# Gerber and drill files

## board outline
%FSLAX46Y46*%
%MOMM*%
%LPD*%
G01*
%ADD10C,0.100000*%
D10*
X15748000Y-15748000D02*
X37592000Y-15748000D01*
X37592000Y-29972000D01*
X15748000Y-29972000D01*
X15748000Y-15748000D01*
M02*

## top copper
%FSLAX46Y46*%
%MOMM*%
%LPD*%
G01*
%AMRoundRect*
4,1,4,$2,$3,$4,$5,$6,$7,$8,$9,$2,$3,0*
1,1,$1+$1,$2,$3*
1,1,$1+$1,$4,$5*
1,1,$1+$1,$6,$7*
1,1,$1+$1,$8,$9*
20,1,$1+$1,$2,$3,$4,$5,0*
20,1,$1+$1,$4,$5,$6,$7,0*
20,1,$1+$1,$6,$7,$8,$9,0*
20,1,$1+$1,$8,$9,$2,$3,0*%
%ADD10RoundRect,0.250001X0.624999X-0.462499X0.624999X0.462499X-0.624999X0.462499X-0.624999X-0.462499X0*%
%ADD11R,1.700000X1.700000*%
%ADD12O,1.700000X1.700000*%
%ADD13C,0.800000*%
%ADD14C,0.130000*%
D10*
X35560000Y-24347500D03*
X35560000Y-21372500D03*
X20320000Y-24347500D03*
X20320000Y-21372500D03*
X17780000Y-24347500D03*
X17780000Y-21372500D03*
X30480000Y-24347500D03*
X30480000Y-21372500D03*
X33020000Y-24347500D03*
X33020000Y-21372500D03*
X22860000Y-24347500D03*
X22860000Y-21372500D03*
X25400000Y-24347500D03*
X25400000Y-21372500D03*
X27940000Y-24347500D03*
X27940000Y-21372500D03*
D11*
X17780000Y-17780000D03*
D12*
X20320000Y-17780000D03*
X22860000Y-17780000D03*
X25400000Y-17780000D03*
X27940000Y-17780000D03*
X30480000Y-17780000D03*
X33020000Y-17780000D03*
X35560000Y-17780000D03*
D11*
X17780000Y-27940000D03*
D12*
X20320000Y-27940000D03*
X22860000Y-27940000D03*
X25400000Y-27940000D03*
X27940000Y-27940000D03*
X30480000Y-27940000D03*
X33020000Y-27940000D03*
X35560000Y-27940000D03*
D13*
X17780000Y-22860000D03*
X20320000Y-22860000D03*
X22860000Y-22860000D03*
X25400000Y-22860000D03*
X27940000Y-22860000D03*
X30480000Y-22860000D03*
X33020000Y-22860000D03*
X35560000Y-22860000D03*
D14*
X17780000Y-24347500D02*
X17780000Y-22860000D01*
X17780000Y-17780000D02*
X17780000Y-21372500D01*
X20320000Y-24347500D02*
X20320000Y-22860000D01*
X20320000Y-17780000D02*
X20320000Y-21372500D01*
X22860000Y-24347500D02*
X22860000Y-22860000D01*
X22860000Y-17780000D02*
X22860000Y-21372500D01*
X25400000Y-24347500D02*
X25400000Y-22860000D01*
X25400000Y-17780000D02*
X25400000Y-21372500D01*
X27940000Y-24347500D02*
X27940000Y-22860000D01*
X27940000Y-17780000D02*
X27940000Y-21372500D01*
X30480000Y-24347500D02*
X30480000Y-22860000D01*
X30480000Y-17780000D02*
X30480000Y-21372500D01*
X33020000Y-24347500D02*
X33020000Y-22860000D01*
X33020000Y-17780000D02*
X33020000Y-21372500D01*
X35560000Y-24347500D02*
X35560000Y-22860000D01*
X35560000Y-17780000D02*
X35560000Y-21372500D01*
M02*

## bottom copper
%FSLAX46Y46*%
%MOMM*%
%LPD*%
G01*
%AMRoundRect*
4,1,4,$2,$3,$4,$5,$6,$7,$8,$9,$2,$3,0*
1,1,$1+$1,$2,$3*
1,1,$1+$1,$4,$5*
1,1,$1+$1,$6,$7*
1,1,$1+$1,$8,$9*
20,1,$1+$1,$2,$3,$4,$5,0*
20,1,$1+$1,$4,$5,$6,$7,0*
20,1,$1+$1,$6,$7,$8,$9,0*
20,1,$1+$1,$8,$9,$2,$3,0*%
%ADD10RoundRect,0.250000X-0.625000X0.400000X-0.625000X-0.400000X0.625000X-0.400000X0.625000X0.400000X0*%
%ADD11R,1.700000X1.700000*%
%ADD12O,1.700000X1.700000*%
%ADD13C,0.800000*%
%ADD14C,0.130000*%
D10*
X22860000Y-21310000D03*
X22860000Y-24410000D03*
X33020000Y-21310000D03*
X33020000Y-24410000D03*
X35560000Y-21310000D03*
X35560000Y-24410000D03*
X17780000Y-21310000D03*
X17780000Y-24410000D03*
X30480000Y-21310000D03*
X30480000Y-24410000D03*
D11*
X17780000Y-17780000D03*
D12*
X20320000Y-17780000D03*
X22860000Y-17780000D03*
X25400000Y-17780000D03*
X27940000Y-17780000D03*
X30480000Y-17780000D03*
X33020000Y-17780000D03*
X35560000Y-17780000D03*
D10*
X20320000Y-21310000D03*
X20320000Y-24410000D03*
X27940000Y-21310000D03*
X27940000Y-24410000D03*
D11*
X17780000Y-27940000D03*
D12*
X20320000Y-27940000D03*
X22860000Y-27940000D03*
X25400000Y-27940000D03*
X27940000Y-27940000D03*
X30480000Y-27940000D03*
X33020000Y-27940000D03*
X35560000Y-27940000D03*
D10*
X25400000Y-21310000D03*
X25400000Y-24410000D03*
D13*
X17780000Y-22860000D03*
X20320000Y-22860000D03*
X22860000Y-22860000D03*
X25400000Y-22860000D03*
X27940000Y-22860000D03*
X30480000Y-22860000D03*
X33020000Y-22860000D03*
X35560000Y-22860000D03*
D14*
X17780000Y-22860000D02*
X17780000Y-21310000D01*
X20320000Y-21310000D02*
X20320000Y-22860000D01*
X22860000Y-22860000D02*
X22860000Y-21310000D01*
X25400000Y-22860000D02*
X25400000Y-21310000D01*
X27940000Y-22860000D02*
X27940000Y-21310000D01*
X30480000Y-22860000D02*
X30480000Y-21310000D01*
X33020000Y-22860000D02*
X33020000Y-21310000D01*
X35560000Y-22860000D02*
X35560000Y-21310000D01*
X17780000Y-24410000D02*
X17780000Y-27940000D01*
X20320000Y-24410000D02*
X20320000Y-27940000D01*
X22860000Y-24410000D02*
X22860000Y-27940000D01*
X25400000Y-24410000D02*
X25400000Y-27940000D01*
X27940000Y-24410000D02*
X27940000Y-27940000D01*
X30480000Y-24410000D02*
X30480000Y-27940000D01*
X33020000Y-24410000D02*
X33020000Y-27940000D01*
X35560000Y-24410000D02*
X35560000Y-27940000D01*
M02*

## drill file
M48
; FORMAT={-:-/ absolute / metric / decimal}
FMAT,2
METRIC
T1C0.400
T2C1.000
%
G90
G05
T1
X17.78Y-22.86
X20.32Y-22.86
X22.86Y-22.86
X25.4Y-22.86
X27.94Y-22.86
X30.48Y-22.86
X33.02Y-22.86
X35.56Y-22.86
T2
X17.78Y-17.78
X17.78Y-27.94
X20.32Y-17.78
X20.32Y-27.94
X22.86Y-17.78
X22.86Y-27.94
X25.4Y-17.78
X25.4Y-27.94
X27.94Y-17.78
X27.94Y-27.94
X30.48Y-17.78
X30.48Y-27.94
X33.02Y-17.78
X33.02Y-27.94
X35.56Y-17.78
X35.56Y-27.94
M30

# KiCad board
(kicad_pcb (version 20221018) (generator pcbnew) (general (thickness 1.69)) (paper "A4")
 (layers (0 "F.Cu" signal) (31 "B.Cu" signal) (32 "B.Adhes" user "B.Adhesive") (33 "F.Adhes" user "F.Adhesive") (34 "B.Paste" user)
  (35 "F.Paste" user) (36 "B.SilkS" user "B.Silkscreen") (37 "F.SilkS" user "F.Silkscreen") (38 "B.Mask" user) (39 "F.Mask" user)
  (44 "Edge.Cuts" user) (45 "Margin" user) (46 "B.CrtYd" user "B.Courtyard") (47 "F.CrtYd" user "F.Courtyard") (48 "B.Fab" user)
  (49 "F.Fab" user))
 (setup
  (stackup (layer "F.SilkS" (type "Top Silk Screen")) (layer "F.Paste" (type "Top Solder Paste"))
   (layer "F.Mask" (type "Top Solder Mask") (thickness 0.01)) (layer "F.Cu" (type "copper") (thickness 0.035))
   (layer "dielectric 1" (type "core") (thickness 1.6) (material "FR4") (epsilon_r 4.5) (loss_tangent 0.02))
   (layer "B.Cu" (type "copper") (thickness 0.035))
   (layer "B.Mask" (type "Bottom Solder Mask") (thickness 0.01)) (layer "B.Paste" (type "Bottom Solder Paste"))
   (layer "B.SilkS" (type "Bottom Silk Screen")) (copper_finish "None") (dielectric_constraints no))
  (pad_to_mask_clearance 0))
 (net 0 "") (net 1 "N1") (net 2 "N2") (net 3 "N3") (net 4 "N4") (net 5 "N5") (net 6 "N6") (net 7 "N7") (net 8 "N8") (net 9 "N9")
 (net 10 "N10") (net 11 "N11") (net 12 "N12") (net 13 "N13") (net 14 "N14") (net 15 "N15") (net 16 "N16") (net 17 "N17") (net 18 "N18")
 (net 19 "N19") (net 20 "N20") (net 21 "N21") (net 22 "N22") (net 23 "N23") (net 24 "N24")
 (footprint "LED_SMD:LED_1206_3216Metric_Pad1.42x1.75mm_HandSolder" (layer "F.Cu") (at 35.56 22.86 90)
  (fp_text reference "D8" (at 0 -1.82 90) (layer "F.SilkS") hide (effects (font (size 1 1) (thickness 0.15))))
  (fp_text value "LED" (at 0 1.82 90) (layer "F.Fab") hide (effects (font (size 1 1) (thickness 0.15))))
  (pad "1" smd roundrect (at -1.4875 0 90) (size 1.425 1.75) (layers "F.Cu" "F.Paste" "F.Mask") (roundrect_rratio 0.1754392982) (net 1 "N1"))
  (pad "2" smd roundrect (at 1.4875 0 90) (size 1.425 1.75) (layers "F.Cu" "F.Paste" "F.Mask") (roundrect_rratio 0.1754392982) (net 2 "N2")))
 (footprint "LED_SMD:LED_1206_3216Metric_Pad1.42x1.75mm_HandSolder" (layer "F.Cu") (at 20.32 22.86 90)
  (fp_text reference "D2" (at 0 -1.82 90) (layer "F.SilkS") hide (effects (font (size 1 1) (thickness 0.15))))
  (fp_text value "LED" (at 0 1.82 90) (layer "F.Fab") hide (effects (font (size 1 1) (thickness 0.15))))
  (pad "1" smd roundrect (at -1.4875 0 90) (size 1.425 1.75) (layers "F.Cu" "F.Paste" "F.Mask") (roundrect_rratio 0.1754392982) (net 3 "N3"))
  (pad "2" smd roundrect (at 1.4875 0 90) (size 1.425 1.75) (layers "F.Cu" "F.Paste" "F.Mask") (roundrect_rratio 0.1754392982) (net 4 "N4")))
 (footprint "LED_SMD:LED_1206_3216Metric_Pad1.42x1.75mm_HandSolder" (layer "F.Cu") (at 17.78 22.86 90)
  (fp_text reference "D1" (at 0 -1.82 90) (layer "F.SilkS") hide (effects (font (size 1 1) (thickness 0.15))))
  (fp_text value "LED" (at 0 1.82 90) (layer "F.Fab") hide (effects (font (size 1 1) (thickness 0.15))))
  (pad "1" smd roundrect (at -1.4875 0 90) (size 1.425 1.75) (layers "F.Cu" "F.Paste" "F.Mask") (roundrect_rratio 0.1754392982) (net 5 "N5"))
  (pad "2" smd roundrect (at 1.4875 0 90) (size 1.425 1.75) (layers "F.Cu" "F.Paste" "F.Mask") (roundrect_rratio 0.1754392982) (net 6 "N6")))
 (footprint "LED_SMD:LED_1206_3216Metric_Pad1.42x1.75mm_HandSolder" (layer "F.Cu") (at 30.48 22.86 90)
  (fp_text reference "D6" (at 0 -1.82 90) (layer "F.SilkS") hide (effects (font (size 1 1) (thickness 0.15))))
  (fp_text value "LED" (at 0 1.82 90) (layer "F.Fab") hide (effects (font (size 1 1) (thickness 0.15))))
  (pad "1" smd roundrect (at -1.4875 0 90) (size 1.425 1.75) (layers "F.Cu" "F.Paste" "F.Mask") (roundrect_rratio 0.1754392982) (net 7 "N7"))
  (pad "2" smd roundrect (at 1.4875 0 90) (size 1.425 1.75) (layers "F.Cu" "F.Paste" "F.Mask") (roundrect_rratio 0.1754392982) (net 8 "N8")))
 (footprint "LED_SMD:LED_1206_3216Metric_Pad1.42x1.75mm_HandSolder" (layer "F.Cu") (at 33.02 22.86 90)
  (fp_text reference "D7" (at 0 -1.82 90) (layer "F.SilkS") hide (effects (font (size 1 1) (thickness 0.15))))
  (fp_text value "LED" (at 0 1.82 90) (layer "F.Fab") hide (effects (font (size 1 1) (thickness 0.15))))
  (pad "1" smd roundrect (at -1.4875 0 90) (size 1.425 1.75) (layers "F.Cu" "F.Paste" "F.Mask") (roundrect_rratio 0.1754392982) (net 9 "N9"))
  (pad "2" smd roundrect (at 1.4875 0 90) (size 1.425 1.75) (layers "F.Cu" "F.Paste" "F.Mask") (roundrect_rratio 0.1754392982)
   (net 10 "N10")))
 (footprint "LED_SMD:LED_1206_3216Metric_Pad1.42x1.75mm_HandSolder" (layer "F.Cu") (at 22.86 22.86 90)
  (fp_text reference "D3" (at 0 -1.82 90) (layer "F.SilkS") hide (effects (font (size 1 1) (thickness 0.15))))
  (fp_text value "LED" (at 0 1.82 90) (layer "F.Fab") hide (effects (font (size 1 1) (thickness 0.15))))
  (pad "1" smd roundrect (at -1.4875 0 90) (size 1.425 1.75) (layers "F.Cu" "F.Paste" "F.Mask") (roundrect_rratio 0.1754392982)
   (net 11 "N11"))
  (pad "2" smd roundrect (at 1.4875 0 90) (size 1.425 1.75) (layers "F.Cu" "F.Paste" "F.Mask") (roundrect_rratio 0.1754392982)
   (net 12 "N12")))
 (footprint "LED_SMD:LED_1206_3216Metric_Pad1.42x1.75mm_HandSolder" (layer "F.Cu") (at 25.4 22.86 90)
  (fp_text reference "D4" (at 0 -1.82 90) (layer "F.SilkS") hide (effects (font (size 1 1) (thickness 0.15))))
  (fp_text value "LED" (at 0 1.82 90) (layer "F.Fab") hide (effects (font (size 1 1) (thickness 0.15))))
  (pad "1" smd roundrect (at -1.4875 0 90) (size 1.425 1.75) (layers "F.Cu" "F.Paste" "F.Mask") (roundrect_rratio 0.1754392982)
   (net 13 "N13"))
  (pad "2" smd roundrect (at 1.4875 0 90) (size 1.425 1.75) (layers "F.Cu" "F.Paste" "F.Mask") (roundrect_rratio 0.1754392982)
   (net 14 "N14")))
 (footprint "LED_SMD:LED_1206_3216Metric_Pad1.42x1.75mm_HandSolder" (layer "F.Cu") (at 27.94 22.86 90)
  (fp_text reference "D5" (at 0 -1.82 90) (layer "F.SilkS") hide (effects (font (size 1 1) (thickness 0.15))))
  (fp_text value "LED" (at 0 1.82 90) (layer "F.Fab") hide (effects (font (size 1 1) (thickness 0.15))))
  (pad "1" smd roundrect (at -1.4875 0 90) (size 1.425 1.75) (layers "F.Cu" "F.Paste" "F.Mask") (roundrect_rratio 0.1754392982)
   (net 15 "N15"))
  (pad "2" smd roundrect (at 1.4875 0 90) (size 1.425 1.75) (layers "F.Cu" "F.Paste" "F.Mask") (roundrect_rratio 0.1754392982)
   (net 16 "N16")))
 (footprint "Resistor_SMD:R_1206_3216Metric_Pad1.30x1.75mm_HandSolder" (layer "B.Cu") (at 22.86 22.86 -90)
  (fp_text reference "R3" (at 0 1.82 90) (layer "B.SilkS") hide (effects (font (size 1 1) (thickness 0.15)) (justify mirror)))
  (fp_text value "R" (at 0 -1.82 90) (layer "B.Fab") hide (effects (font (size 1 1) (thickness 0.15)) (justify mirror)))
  (pad "1" smd roundrect (at -1.55 0 270) (size 1.3 1.75) (layers "B.Cu" "B.Paste" "B.Mask") (roundrect_rratio 0.1923076923) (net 11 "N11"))
  (pad "2" smd roundrect (at 1.55 0 270) (size 1.3 1.75) (layers "B.Cu" "B.Paste" "B.Mask") (roundrect_rratio 0.1923076923) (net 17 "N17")))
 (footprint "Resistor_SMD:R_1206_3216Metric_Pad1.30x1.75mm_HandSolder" (layer "B.Cu") (at 33.02 22.86 -90)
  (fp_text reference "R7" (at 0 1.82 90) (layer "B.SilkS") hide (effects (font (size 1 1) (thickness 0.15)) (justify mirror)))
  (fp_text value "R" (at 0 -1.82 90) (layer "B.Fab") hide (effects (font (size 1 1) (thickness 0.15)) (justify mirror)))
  (pad "1" smd roundrect (at -1.55 0 270) (size 1.3 1.75) (layers "B.Cu" "B.Paste" "B.Mask") (roundrect_rratio 0.1923076923) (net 9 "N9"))
  (pad "2" smd roundrect (at 1.55 0 270) (size 1.3 1.75) (layers "B.Cu" "B.Paste" "B.Mask") (roundrect_rratio 0.1923076923) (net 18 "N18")))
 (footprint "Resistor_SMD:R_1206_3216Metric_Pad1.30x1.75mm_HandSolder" (layer "B.Cu") (at 35.56 22.86 -90)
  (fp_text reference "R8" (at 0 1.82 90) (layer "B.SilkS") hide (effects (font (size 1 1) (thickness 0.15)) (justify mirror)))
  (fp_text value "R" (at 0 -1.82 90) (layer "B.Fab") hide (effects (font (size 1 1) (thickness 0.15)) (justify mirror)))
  (pad "1" smd roundrect (at -1.55 0 270) (size 1.3 1.75) (layers "B.Cu" "B.Paste" "B.Mask") (roundrect_rratio 0.1923076923) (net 1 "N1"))
  (pad "2" smd roundrect (at 1.55 0 270) (size 1.3 1.75) (layers "B.Cu" "B.Paste" "B.Mask") (roundrect_rratio 0.1923076923) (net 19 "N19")))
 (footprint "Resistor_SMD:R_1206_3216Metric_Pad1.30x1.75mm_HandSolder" (layer "B.Cu") (at 17.78 22.86 -90)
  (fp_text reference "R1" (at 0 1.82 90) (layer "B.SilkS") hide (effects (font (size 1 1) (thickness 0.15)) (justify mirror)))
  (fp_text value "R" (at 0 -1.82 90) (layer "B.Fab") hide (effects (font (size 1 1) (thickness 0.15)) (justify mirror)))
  (pad "1" smd roundrect (at -1.55 0 270) (size 1.3 1.75) (layers "B.Cu" "B.Paste" "B.Mask") (roundrect_rratio 0.1923076923) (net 5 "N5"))
  (pad "2" smd roundrect (at 1.55 0 270) (size 1.3 1.75) (layers "B.Cu" "B.Paste" "B.Mask") (roundrect_rratio 0.1923076923) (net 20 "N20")))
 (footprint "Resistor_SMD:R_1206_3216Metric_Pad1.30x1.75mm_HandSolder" (layer "B.Cu") (at 30.48 22.86 -90)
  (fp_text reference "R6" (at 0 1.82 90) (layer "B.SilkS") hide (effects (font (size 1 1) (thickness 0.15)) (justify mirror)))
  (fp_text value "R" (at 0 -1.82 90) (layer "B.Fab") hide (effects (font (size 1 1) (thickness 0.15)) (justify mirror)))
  (pad "1" smd roundrect (at -1.55 0 270) (size 1.3 1.75) (layers "B.Cu" "B.Paste" "B.Mask") (roundrect_rratio 0.1923076923) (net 7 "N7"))
  (pad "2" smd roundrect (at 1.55 0 270) (size 1.3 1.75) (layers "B.Cu" "B.Paste" "B.Mask") (roundrect_rratio 0.1923076923) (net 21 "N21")))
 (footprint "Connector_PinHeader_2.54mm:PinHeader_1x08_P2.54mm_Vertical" (layer "B.Cu") (at 17.78 17.78 -90)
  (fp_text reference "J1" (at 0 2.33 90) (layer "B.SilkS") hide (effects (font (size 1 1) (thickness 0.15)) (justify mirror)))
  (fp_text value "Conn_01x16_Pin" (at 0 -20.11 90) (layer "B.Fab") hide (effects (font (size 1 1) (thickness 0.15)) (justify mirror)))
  (pad "1" thru_hole rect (at 0 0 270) (size 1.7 1.7) (drill 1) (layers "*.Cu" "*.Mask") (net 6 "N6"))
  (pad "2" thru_hole oval (at 0 -2.54 270) (size 1.7 1.7) (drill 1) (layers "*.Cu" "*.Mask") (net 4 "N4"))
  (pad "3" thru_hole oval (at 0 -5.08 270) (size 1.7 1.7) (drill 1) (layers "*.Cu" "*.Mask") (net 12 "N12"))
  (pad "4" thru_hole oval (at 0 -7.62 270) (size 1.7 1.7) (drill 1) (layers "*.Cu" "*.Mask") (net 14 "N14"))
  (pad "5" thru_hole oval (at 0 -10.16 270) (size 1.7 1.7) (drill 1) (layers "*.Cu" "*.Mask") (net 16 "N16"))
  (pad "6" thru_hole oval (at 0 -12.7 270) (size 1.7 1.7) (drill 1) (layers "*.Cu" "*.Mask") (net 8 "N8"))
  (pad "7" thru_hole oval (at 0 -15.24 270) (size 1.7 1.7) (drill 1) (layers "*.Cu" "*.Mask") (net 10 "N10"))
  (pad "8" thru_hole oval (at 0 -17.78 270) (size 1.7 1.7) (drill 1) (layers "*.Cu" "*.Mask") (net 2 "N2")))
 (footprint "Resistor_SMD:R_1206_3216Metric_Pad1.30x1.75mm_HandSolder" (layer "B.Cu") (at 20.32 22.86 -90)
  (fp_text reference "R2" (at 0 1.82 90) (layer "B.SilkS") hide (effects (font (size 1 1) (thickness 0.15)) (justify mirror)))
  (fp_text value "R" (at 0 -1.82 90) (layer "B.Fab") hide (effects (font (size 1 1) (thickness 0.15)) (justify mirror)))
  (pad "1" smd roundrect (at -1.55 0 270) (size 1.3 1.75) (layers "B.Cu" "B.Paste" "B.Mask") (roundrect_rratio 0.1923076923) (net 3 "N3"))
  (pad "2" smd roundrect (at 1.55 0 270) (size 1.3 1.75) (layers "B.Cu" "B.Paste" "B.Mask") (roundrect_rratio 0.1923076923) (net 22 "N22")))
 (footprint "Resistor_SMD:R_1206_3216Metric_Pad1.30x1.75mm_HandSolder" (layer "B.Cu") (at 27.94 22.86 -90)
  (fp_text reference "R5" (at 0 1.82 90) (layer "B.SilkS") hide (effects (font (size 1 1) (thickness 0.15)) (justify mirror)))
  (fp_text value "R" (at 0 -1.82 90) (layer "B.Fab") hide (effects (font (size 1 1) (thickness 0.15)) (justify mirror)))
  (pad "1" smd roundrect (at -1.55 0 270) (size 1.3 1.75) (layers "B.Cu" "B.Paste" "B.Mask") (roundrect_rratio 0.1923076923) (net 15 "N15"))
  (pad "2" smd roundrect (at 1.55 0 270) (size 1.3 1.75) (layers "B.Cu" "B.Paste" "B.Mask") (roundrect_rratio 0.1923076923) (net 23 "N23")))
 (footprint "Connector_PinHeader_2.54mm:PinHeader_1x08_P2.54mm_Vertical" (layer "B.Cu") (at 17.78 27.94 -90)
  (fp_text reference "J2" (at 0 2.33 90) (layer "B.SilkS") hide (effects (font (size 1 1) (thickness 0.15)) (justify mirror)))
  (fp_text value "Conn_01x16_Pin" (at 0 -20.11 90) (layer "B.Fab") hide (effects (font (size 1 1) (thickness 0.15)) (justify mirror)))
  (pad "1" thru_hole rect (at 0 0 270) (size 1.7 1.7) (drill 1) (layers "*.Cu" "*.Mask") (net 20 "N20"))
  (pad "2" thru_hole oval (at 0 -2.54 270) (size 1.7 1.7) (drill 1) (layers "*.Cu" "*.Mask") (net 22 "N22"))
  (pad "3" thru_hole oval (at 0 -5.08 270) (size 1.7 1.7) (drill 1) (layers "*.Cu" "*.Mask") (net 17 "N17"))
  (pad "4" thru_hole oval (at 0 -7.62 270) (size 1.7 1.7) (drill 1) (layers "*.Cu" "*.Mask") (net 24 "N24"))
  (pad "5" thru_hole oval (at 0 -10.16 270) (size 1.7 1.7) (drill 1) (layers "*.Cu" "*.Mask") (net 23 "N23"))
  (pad "6" thru_hole oval (at 0 -12.7 270) (size 1.7 1.7) (drill 1) (layers "*.Cu" "*.Mask") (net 21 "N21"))
  (pad "7" thru_hole oval (at 0 -15.24 270) (size 1.7 1.7) (drill 1) (layers "*.Cu" "*.Mask") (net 18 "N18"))
  (pad "8" thru_hole oval (at 0 -17.78 270) (size 1.7 1.7) (drill 1) (layers "*.Cu" "*.Mask") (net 19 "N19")))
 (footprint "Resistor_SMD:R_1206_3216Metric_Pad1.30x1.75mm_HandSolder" (layer "B.Cu") (at 25.4 22.86 -90)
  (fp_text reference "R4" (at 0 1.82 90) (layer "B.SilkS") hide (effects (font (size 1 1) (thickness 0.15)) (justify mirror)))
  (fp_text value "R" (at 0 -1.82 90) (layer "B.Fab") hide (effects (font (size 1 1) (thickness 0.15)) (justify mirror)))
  (pad "1" smd roundrect (at -1.55 0 270) (size 1.3 1.75) (layers "B.Cu" "B.Paste" "B.Mask") (roundrect_rratio 0.1923076923) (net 13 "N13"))
  (pad "2" smd roundrect (at 1.55 0 270) (size 1.3 1.75) (layers "B.Cu" "B.Paste" "B.Mask") (roundrect_rratio 0.1923076923) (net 24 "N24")))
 (gr_rect (start 15.748 15.748) (end 37.592 29.972) (stroke (width 0.1) (type default)) (fill none) (layer "Edge.Cuts"))
 (segment (start 17.78 24.3475) (end 17.78 22.86) (width 0.13) (layer "F.Cu") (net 5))
 (via (at 17.78 22.86) (size 0.8) (drill 0.4) (layers "F.Cu" "B.Cu") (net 5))
 (segment (start 17.78 22.86) (end 17.78 21.31) (width 0.13) (layer "B.Cu") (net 5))
 (segment (start 17.78 17.78) (end 17.78 21.3725) (width 0.13) (layer "F.Cu") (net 6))
 (segment (start 20.32 24.3475) (end 20.32 22.86) (width 0.13) (layer "F.Cu") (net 3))
 (via (at 20.32 22.86) (size 0.8) (drill 0.4) (layers "F.Cu" "B.Cu") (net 3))
 (segment (start 20.32 21.31) (end 20.32 22.86) (width 0.13) (layer "B.Cu") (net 3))
 (segment (start 20.32 17.78) (end 20.32 21.3725) (width 0.13) (layer "F.Cu") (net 4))
 (segment (start 22.86 24.3475) (end 22.86 22.86) (width 0.13) (layer "F.Cu") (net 11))
 (via (at 22.86 22.86) (size 0.8) (drill 0.4) (layers "F.Cu" "B.Cu") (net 11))
 (segment (start 22.86 22.86) (end 22.86 21.31) (width 0.13) (layer "B.Cu") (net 11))
 (segment (start 22.86 17.78) (end 22.86 21.3725) (width 0.13) (layer "F.Cu") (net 12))
 (segment (start 25.4 24.3475) (end 25.4 22.86) (width 0.13) (layer "F.Cu") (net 13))
 (via (at 25.4 22.86) (size 0.8) (drill 0.4) (layers "F.Cu" "B.Cu") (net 13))
 (segment (start 25.4 22.86) (end 25.4 21.31) (width 0.13) (layer "B.Cu") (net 13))
 (segment (start 25.4 17.78) (end 25.4 21.3725) (width 0.13) (layer "F.Cu") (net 14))
 (segment (start 27.94 24.3475) (end 27.94 22.86) (width 0.13) (layer "F.Cu") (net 15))
 (via (at 27.94 22.86) (size 0.8) (drill 0.4) (layers "F.Cu" "B.Cu") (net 15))
 (segment (start 27.94 22.86) (end 27.94 21.31) (width 0.13) (layer "B.Cu") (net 15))
 (segment (start 27.94 17.78) (end 27.94 21.3725) (width 0.13) (layer "F.Cu") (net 16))
 (segment (start 30.48 24.3475) (end 30.48 22.86) (width 0.13) (layer "F.Cu") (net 7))
 (via (at 30.48 22.86) (size 0.8) (drill 0.4) (layers "F.Cu" "B.Cu") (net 7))
 (segment (start 30.48 22.86) (end 30.48 21.31) (width 0.13) (layer "B.Cu") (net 7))
 (segment (start 30.48 17.78) (end 30.48 21.3725) (width 0.13) (layer "F.Cu") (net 8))
 (segment (start 33.02 24.3475) (end 33.02 22.86) (width 0.13) (layer "F.Cu") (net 9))
 (via (at 33.02 22.86) (size 0.8) (drill 0.4) (layers "F.Cu" "B.Cu") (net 9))
 (segment (start 33.02 22.86) (end 33.02 21.31) (width 0.13) (layer "B.Cu") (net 9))
 (segment (start 33.02 17.78) (end 33.02 21.3725) (width 0.13) (layer "F.Cu") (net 10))
 (segment (start 35.56 24.3475) (end 35.56 22.86) (width 0.13) (layer "F.Cu") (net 1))
 (via (at 35.56 22.86) (size 0.8) (drill 0.4) (layers "F.Cu" "B.Cu") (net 1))
 (segment (start 35.56 22.86) (end 35.56 21.31) (width 0.13) (layer "B.Cu") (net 1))
 (segment (start 35.56 17.78) (end 35.56 21.3725) (width 0.13) (layer "F.Cu") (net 2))
 (segment (start 17.78 24.41) (end 17.78 27.94) (width 0.13) (layer "B.Cu") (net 20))
 (segment (start 20.32 24.41) (end 20.32 27.94) (width 0.13) (layer "B.Cu") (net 22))
 (segment (start 22.86 24.41) (end 22.86 27.94) (width 0.13) (layer "B.Cu") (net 17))
 (segment (start 25.4 24.41) (end 25.4 27.94) (width 0.13) (layer "B.Cu") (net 24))
 (segment (start 27.94 24.41) (end 27.94 27.94) (width 0.13) (layer "B.Cu") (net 23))
 (segment (start 30.48 24.41) (end 30.48 27.94) (width 0.13) (layer "B.Cu") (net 21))
 (segment (start 33.02 24.41) (end 33.02 27.94) (width 0.13) (layer "B.Cu") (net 18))
 (segment (start 35.56 24.41) (end 35.56 27.94) (width 0.13) (layer "B.Cu") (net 19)))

